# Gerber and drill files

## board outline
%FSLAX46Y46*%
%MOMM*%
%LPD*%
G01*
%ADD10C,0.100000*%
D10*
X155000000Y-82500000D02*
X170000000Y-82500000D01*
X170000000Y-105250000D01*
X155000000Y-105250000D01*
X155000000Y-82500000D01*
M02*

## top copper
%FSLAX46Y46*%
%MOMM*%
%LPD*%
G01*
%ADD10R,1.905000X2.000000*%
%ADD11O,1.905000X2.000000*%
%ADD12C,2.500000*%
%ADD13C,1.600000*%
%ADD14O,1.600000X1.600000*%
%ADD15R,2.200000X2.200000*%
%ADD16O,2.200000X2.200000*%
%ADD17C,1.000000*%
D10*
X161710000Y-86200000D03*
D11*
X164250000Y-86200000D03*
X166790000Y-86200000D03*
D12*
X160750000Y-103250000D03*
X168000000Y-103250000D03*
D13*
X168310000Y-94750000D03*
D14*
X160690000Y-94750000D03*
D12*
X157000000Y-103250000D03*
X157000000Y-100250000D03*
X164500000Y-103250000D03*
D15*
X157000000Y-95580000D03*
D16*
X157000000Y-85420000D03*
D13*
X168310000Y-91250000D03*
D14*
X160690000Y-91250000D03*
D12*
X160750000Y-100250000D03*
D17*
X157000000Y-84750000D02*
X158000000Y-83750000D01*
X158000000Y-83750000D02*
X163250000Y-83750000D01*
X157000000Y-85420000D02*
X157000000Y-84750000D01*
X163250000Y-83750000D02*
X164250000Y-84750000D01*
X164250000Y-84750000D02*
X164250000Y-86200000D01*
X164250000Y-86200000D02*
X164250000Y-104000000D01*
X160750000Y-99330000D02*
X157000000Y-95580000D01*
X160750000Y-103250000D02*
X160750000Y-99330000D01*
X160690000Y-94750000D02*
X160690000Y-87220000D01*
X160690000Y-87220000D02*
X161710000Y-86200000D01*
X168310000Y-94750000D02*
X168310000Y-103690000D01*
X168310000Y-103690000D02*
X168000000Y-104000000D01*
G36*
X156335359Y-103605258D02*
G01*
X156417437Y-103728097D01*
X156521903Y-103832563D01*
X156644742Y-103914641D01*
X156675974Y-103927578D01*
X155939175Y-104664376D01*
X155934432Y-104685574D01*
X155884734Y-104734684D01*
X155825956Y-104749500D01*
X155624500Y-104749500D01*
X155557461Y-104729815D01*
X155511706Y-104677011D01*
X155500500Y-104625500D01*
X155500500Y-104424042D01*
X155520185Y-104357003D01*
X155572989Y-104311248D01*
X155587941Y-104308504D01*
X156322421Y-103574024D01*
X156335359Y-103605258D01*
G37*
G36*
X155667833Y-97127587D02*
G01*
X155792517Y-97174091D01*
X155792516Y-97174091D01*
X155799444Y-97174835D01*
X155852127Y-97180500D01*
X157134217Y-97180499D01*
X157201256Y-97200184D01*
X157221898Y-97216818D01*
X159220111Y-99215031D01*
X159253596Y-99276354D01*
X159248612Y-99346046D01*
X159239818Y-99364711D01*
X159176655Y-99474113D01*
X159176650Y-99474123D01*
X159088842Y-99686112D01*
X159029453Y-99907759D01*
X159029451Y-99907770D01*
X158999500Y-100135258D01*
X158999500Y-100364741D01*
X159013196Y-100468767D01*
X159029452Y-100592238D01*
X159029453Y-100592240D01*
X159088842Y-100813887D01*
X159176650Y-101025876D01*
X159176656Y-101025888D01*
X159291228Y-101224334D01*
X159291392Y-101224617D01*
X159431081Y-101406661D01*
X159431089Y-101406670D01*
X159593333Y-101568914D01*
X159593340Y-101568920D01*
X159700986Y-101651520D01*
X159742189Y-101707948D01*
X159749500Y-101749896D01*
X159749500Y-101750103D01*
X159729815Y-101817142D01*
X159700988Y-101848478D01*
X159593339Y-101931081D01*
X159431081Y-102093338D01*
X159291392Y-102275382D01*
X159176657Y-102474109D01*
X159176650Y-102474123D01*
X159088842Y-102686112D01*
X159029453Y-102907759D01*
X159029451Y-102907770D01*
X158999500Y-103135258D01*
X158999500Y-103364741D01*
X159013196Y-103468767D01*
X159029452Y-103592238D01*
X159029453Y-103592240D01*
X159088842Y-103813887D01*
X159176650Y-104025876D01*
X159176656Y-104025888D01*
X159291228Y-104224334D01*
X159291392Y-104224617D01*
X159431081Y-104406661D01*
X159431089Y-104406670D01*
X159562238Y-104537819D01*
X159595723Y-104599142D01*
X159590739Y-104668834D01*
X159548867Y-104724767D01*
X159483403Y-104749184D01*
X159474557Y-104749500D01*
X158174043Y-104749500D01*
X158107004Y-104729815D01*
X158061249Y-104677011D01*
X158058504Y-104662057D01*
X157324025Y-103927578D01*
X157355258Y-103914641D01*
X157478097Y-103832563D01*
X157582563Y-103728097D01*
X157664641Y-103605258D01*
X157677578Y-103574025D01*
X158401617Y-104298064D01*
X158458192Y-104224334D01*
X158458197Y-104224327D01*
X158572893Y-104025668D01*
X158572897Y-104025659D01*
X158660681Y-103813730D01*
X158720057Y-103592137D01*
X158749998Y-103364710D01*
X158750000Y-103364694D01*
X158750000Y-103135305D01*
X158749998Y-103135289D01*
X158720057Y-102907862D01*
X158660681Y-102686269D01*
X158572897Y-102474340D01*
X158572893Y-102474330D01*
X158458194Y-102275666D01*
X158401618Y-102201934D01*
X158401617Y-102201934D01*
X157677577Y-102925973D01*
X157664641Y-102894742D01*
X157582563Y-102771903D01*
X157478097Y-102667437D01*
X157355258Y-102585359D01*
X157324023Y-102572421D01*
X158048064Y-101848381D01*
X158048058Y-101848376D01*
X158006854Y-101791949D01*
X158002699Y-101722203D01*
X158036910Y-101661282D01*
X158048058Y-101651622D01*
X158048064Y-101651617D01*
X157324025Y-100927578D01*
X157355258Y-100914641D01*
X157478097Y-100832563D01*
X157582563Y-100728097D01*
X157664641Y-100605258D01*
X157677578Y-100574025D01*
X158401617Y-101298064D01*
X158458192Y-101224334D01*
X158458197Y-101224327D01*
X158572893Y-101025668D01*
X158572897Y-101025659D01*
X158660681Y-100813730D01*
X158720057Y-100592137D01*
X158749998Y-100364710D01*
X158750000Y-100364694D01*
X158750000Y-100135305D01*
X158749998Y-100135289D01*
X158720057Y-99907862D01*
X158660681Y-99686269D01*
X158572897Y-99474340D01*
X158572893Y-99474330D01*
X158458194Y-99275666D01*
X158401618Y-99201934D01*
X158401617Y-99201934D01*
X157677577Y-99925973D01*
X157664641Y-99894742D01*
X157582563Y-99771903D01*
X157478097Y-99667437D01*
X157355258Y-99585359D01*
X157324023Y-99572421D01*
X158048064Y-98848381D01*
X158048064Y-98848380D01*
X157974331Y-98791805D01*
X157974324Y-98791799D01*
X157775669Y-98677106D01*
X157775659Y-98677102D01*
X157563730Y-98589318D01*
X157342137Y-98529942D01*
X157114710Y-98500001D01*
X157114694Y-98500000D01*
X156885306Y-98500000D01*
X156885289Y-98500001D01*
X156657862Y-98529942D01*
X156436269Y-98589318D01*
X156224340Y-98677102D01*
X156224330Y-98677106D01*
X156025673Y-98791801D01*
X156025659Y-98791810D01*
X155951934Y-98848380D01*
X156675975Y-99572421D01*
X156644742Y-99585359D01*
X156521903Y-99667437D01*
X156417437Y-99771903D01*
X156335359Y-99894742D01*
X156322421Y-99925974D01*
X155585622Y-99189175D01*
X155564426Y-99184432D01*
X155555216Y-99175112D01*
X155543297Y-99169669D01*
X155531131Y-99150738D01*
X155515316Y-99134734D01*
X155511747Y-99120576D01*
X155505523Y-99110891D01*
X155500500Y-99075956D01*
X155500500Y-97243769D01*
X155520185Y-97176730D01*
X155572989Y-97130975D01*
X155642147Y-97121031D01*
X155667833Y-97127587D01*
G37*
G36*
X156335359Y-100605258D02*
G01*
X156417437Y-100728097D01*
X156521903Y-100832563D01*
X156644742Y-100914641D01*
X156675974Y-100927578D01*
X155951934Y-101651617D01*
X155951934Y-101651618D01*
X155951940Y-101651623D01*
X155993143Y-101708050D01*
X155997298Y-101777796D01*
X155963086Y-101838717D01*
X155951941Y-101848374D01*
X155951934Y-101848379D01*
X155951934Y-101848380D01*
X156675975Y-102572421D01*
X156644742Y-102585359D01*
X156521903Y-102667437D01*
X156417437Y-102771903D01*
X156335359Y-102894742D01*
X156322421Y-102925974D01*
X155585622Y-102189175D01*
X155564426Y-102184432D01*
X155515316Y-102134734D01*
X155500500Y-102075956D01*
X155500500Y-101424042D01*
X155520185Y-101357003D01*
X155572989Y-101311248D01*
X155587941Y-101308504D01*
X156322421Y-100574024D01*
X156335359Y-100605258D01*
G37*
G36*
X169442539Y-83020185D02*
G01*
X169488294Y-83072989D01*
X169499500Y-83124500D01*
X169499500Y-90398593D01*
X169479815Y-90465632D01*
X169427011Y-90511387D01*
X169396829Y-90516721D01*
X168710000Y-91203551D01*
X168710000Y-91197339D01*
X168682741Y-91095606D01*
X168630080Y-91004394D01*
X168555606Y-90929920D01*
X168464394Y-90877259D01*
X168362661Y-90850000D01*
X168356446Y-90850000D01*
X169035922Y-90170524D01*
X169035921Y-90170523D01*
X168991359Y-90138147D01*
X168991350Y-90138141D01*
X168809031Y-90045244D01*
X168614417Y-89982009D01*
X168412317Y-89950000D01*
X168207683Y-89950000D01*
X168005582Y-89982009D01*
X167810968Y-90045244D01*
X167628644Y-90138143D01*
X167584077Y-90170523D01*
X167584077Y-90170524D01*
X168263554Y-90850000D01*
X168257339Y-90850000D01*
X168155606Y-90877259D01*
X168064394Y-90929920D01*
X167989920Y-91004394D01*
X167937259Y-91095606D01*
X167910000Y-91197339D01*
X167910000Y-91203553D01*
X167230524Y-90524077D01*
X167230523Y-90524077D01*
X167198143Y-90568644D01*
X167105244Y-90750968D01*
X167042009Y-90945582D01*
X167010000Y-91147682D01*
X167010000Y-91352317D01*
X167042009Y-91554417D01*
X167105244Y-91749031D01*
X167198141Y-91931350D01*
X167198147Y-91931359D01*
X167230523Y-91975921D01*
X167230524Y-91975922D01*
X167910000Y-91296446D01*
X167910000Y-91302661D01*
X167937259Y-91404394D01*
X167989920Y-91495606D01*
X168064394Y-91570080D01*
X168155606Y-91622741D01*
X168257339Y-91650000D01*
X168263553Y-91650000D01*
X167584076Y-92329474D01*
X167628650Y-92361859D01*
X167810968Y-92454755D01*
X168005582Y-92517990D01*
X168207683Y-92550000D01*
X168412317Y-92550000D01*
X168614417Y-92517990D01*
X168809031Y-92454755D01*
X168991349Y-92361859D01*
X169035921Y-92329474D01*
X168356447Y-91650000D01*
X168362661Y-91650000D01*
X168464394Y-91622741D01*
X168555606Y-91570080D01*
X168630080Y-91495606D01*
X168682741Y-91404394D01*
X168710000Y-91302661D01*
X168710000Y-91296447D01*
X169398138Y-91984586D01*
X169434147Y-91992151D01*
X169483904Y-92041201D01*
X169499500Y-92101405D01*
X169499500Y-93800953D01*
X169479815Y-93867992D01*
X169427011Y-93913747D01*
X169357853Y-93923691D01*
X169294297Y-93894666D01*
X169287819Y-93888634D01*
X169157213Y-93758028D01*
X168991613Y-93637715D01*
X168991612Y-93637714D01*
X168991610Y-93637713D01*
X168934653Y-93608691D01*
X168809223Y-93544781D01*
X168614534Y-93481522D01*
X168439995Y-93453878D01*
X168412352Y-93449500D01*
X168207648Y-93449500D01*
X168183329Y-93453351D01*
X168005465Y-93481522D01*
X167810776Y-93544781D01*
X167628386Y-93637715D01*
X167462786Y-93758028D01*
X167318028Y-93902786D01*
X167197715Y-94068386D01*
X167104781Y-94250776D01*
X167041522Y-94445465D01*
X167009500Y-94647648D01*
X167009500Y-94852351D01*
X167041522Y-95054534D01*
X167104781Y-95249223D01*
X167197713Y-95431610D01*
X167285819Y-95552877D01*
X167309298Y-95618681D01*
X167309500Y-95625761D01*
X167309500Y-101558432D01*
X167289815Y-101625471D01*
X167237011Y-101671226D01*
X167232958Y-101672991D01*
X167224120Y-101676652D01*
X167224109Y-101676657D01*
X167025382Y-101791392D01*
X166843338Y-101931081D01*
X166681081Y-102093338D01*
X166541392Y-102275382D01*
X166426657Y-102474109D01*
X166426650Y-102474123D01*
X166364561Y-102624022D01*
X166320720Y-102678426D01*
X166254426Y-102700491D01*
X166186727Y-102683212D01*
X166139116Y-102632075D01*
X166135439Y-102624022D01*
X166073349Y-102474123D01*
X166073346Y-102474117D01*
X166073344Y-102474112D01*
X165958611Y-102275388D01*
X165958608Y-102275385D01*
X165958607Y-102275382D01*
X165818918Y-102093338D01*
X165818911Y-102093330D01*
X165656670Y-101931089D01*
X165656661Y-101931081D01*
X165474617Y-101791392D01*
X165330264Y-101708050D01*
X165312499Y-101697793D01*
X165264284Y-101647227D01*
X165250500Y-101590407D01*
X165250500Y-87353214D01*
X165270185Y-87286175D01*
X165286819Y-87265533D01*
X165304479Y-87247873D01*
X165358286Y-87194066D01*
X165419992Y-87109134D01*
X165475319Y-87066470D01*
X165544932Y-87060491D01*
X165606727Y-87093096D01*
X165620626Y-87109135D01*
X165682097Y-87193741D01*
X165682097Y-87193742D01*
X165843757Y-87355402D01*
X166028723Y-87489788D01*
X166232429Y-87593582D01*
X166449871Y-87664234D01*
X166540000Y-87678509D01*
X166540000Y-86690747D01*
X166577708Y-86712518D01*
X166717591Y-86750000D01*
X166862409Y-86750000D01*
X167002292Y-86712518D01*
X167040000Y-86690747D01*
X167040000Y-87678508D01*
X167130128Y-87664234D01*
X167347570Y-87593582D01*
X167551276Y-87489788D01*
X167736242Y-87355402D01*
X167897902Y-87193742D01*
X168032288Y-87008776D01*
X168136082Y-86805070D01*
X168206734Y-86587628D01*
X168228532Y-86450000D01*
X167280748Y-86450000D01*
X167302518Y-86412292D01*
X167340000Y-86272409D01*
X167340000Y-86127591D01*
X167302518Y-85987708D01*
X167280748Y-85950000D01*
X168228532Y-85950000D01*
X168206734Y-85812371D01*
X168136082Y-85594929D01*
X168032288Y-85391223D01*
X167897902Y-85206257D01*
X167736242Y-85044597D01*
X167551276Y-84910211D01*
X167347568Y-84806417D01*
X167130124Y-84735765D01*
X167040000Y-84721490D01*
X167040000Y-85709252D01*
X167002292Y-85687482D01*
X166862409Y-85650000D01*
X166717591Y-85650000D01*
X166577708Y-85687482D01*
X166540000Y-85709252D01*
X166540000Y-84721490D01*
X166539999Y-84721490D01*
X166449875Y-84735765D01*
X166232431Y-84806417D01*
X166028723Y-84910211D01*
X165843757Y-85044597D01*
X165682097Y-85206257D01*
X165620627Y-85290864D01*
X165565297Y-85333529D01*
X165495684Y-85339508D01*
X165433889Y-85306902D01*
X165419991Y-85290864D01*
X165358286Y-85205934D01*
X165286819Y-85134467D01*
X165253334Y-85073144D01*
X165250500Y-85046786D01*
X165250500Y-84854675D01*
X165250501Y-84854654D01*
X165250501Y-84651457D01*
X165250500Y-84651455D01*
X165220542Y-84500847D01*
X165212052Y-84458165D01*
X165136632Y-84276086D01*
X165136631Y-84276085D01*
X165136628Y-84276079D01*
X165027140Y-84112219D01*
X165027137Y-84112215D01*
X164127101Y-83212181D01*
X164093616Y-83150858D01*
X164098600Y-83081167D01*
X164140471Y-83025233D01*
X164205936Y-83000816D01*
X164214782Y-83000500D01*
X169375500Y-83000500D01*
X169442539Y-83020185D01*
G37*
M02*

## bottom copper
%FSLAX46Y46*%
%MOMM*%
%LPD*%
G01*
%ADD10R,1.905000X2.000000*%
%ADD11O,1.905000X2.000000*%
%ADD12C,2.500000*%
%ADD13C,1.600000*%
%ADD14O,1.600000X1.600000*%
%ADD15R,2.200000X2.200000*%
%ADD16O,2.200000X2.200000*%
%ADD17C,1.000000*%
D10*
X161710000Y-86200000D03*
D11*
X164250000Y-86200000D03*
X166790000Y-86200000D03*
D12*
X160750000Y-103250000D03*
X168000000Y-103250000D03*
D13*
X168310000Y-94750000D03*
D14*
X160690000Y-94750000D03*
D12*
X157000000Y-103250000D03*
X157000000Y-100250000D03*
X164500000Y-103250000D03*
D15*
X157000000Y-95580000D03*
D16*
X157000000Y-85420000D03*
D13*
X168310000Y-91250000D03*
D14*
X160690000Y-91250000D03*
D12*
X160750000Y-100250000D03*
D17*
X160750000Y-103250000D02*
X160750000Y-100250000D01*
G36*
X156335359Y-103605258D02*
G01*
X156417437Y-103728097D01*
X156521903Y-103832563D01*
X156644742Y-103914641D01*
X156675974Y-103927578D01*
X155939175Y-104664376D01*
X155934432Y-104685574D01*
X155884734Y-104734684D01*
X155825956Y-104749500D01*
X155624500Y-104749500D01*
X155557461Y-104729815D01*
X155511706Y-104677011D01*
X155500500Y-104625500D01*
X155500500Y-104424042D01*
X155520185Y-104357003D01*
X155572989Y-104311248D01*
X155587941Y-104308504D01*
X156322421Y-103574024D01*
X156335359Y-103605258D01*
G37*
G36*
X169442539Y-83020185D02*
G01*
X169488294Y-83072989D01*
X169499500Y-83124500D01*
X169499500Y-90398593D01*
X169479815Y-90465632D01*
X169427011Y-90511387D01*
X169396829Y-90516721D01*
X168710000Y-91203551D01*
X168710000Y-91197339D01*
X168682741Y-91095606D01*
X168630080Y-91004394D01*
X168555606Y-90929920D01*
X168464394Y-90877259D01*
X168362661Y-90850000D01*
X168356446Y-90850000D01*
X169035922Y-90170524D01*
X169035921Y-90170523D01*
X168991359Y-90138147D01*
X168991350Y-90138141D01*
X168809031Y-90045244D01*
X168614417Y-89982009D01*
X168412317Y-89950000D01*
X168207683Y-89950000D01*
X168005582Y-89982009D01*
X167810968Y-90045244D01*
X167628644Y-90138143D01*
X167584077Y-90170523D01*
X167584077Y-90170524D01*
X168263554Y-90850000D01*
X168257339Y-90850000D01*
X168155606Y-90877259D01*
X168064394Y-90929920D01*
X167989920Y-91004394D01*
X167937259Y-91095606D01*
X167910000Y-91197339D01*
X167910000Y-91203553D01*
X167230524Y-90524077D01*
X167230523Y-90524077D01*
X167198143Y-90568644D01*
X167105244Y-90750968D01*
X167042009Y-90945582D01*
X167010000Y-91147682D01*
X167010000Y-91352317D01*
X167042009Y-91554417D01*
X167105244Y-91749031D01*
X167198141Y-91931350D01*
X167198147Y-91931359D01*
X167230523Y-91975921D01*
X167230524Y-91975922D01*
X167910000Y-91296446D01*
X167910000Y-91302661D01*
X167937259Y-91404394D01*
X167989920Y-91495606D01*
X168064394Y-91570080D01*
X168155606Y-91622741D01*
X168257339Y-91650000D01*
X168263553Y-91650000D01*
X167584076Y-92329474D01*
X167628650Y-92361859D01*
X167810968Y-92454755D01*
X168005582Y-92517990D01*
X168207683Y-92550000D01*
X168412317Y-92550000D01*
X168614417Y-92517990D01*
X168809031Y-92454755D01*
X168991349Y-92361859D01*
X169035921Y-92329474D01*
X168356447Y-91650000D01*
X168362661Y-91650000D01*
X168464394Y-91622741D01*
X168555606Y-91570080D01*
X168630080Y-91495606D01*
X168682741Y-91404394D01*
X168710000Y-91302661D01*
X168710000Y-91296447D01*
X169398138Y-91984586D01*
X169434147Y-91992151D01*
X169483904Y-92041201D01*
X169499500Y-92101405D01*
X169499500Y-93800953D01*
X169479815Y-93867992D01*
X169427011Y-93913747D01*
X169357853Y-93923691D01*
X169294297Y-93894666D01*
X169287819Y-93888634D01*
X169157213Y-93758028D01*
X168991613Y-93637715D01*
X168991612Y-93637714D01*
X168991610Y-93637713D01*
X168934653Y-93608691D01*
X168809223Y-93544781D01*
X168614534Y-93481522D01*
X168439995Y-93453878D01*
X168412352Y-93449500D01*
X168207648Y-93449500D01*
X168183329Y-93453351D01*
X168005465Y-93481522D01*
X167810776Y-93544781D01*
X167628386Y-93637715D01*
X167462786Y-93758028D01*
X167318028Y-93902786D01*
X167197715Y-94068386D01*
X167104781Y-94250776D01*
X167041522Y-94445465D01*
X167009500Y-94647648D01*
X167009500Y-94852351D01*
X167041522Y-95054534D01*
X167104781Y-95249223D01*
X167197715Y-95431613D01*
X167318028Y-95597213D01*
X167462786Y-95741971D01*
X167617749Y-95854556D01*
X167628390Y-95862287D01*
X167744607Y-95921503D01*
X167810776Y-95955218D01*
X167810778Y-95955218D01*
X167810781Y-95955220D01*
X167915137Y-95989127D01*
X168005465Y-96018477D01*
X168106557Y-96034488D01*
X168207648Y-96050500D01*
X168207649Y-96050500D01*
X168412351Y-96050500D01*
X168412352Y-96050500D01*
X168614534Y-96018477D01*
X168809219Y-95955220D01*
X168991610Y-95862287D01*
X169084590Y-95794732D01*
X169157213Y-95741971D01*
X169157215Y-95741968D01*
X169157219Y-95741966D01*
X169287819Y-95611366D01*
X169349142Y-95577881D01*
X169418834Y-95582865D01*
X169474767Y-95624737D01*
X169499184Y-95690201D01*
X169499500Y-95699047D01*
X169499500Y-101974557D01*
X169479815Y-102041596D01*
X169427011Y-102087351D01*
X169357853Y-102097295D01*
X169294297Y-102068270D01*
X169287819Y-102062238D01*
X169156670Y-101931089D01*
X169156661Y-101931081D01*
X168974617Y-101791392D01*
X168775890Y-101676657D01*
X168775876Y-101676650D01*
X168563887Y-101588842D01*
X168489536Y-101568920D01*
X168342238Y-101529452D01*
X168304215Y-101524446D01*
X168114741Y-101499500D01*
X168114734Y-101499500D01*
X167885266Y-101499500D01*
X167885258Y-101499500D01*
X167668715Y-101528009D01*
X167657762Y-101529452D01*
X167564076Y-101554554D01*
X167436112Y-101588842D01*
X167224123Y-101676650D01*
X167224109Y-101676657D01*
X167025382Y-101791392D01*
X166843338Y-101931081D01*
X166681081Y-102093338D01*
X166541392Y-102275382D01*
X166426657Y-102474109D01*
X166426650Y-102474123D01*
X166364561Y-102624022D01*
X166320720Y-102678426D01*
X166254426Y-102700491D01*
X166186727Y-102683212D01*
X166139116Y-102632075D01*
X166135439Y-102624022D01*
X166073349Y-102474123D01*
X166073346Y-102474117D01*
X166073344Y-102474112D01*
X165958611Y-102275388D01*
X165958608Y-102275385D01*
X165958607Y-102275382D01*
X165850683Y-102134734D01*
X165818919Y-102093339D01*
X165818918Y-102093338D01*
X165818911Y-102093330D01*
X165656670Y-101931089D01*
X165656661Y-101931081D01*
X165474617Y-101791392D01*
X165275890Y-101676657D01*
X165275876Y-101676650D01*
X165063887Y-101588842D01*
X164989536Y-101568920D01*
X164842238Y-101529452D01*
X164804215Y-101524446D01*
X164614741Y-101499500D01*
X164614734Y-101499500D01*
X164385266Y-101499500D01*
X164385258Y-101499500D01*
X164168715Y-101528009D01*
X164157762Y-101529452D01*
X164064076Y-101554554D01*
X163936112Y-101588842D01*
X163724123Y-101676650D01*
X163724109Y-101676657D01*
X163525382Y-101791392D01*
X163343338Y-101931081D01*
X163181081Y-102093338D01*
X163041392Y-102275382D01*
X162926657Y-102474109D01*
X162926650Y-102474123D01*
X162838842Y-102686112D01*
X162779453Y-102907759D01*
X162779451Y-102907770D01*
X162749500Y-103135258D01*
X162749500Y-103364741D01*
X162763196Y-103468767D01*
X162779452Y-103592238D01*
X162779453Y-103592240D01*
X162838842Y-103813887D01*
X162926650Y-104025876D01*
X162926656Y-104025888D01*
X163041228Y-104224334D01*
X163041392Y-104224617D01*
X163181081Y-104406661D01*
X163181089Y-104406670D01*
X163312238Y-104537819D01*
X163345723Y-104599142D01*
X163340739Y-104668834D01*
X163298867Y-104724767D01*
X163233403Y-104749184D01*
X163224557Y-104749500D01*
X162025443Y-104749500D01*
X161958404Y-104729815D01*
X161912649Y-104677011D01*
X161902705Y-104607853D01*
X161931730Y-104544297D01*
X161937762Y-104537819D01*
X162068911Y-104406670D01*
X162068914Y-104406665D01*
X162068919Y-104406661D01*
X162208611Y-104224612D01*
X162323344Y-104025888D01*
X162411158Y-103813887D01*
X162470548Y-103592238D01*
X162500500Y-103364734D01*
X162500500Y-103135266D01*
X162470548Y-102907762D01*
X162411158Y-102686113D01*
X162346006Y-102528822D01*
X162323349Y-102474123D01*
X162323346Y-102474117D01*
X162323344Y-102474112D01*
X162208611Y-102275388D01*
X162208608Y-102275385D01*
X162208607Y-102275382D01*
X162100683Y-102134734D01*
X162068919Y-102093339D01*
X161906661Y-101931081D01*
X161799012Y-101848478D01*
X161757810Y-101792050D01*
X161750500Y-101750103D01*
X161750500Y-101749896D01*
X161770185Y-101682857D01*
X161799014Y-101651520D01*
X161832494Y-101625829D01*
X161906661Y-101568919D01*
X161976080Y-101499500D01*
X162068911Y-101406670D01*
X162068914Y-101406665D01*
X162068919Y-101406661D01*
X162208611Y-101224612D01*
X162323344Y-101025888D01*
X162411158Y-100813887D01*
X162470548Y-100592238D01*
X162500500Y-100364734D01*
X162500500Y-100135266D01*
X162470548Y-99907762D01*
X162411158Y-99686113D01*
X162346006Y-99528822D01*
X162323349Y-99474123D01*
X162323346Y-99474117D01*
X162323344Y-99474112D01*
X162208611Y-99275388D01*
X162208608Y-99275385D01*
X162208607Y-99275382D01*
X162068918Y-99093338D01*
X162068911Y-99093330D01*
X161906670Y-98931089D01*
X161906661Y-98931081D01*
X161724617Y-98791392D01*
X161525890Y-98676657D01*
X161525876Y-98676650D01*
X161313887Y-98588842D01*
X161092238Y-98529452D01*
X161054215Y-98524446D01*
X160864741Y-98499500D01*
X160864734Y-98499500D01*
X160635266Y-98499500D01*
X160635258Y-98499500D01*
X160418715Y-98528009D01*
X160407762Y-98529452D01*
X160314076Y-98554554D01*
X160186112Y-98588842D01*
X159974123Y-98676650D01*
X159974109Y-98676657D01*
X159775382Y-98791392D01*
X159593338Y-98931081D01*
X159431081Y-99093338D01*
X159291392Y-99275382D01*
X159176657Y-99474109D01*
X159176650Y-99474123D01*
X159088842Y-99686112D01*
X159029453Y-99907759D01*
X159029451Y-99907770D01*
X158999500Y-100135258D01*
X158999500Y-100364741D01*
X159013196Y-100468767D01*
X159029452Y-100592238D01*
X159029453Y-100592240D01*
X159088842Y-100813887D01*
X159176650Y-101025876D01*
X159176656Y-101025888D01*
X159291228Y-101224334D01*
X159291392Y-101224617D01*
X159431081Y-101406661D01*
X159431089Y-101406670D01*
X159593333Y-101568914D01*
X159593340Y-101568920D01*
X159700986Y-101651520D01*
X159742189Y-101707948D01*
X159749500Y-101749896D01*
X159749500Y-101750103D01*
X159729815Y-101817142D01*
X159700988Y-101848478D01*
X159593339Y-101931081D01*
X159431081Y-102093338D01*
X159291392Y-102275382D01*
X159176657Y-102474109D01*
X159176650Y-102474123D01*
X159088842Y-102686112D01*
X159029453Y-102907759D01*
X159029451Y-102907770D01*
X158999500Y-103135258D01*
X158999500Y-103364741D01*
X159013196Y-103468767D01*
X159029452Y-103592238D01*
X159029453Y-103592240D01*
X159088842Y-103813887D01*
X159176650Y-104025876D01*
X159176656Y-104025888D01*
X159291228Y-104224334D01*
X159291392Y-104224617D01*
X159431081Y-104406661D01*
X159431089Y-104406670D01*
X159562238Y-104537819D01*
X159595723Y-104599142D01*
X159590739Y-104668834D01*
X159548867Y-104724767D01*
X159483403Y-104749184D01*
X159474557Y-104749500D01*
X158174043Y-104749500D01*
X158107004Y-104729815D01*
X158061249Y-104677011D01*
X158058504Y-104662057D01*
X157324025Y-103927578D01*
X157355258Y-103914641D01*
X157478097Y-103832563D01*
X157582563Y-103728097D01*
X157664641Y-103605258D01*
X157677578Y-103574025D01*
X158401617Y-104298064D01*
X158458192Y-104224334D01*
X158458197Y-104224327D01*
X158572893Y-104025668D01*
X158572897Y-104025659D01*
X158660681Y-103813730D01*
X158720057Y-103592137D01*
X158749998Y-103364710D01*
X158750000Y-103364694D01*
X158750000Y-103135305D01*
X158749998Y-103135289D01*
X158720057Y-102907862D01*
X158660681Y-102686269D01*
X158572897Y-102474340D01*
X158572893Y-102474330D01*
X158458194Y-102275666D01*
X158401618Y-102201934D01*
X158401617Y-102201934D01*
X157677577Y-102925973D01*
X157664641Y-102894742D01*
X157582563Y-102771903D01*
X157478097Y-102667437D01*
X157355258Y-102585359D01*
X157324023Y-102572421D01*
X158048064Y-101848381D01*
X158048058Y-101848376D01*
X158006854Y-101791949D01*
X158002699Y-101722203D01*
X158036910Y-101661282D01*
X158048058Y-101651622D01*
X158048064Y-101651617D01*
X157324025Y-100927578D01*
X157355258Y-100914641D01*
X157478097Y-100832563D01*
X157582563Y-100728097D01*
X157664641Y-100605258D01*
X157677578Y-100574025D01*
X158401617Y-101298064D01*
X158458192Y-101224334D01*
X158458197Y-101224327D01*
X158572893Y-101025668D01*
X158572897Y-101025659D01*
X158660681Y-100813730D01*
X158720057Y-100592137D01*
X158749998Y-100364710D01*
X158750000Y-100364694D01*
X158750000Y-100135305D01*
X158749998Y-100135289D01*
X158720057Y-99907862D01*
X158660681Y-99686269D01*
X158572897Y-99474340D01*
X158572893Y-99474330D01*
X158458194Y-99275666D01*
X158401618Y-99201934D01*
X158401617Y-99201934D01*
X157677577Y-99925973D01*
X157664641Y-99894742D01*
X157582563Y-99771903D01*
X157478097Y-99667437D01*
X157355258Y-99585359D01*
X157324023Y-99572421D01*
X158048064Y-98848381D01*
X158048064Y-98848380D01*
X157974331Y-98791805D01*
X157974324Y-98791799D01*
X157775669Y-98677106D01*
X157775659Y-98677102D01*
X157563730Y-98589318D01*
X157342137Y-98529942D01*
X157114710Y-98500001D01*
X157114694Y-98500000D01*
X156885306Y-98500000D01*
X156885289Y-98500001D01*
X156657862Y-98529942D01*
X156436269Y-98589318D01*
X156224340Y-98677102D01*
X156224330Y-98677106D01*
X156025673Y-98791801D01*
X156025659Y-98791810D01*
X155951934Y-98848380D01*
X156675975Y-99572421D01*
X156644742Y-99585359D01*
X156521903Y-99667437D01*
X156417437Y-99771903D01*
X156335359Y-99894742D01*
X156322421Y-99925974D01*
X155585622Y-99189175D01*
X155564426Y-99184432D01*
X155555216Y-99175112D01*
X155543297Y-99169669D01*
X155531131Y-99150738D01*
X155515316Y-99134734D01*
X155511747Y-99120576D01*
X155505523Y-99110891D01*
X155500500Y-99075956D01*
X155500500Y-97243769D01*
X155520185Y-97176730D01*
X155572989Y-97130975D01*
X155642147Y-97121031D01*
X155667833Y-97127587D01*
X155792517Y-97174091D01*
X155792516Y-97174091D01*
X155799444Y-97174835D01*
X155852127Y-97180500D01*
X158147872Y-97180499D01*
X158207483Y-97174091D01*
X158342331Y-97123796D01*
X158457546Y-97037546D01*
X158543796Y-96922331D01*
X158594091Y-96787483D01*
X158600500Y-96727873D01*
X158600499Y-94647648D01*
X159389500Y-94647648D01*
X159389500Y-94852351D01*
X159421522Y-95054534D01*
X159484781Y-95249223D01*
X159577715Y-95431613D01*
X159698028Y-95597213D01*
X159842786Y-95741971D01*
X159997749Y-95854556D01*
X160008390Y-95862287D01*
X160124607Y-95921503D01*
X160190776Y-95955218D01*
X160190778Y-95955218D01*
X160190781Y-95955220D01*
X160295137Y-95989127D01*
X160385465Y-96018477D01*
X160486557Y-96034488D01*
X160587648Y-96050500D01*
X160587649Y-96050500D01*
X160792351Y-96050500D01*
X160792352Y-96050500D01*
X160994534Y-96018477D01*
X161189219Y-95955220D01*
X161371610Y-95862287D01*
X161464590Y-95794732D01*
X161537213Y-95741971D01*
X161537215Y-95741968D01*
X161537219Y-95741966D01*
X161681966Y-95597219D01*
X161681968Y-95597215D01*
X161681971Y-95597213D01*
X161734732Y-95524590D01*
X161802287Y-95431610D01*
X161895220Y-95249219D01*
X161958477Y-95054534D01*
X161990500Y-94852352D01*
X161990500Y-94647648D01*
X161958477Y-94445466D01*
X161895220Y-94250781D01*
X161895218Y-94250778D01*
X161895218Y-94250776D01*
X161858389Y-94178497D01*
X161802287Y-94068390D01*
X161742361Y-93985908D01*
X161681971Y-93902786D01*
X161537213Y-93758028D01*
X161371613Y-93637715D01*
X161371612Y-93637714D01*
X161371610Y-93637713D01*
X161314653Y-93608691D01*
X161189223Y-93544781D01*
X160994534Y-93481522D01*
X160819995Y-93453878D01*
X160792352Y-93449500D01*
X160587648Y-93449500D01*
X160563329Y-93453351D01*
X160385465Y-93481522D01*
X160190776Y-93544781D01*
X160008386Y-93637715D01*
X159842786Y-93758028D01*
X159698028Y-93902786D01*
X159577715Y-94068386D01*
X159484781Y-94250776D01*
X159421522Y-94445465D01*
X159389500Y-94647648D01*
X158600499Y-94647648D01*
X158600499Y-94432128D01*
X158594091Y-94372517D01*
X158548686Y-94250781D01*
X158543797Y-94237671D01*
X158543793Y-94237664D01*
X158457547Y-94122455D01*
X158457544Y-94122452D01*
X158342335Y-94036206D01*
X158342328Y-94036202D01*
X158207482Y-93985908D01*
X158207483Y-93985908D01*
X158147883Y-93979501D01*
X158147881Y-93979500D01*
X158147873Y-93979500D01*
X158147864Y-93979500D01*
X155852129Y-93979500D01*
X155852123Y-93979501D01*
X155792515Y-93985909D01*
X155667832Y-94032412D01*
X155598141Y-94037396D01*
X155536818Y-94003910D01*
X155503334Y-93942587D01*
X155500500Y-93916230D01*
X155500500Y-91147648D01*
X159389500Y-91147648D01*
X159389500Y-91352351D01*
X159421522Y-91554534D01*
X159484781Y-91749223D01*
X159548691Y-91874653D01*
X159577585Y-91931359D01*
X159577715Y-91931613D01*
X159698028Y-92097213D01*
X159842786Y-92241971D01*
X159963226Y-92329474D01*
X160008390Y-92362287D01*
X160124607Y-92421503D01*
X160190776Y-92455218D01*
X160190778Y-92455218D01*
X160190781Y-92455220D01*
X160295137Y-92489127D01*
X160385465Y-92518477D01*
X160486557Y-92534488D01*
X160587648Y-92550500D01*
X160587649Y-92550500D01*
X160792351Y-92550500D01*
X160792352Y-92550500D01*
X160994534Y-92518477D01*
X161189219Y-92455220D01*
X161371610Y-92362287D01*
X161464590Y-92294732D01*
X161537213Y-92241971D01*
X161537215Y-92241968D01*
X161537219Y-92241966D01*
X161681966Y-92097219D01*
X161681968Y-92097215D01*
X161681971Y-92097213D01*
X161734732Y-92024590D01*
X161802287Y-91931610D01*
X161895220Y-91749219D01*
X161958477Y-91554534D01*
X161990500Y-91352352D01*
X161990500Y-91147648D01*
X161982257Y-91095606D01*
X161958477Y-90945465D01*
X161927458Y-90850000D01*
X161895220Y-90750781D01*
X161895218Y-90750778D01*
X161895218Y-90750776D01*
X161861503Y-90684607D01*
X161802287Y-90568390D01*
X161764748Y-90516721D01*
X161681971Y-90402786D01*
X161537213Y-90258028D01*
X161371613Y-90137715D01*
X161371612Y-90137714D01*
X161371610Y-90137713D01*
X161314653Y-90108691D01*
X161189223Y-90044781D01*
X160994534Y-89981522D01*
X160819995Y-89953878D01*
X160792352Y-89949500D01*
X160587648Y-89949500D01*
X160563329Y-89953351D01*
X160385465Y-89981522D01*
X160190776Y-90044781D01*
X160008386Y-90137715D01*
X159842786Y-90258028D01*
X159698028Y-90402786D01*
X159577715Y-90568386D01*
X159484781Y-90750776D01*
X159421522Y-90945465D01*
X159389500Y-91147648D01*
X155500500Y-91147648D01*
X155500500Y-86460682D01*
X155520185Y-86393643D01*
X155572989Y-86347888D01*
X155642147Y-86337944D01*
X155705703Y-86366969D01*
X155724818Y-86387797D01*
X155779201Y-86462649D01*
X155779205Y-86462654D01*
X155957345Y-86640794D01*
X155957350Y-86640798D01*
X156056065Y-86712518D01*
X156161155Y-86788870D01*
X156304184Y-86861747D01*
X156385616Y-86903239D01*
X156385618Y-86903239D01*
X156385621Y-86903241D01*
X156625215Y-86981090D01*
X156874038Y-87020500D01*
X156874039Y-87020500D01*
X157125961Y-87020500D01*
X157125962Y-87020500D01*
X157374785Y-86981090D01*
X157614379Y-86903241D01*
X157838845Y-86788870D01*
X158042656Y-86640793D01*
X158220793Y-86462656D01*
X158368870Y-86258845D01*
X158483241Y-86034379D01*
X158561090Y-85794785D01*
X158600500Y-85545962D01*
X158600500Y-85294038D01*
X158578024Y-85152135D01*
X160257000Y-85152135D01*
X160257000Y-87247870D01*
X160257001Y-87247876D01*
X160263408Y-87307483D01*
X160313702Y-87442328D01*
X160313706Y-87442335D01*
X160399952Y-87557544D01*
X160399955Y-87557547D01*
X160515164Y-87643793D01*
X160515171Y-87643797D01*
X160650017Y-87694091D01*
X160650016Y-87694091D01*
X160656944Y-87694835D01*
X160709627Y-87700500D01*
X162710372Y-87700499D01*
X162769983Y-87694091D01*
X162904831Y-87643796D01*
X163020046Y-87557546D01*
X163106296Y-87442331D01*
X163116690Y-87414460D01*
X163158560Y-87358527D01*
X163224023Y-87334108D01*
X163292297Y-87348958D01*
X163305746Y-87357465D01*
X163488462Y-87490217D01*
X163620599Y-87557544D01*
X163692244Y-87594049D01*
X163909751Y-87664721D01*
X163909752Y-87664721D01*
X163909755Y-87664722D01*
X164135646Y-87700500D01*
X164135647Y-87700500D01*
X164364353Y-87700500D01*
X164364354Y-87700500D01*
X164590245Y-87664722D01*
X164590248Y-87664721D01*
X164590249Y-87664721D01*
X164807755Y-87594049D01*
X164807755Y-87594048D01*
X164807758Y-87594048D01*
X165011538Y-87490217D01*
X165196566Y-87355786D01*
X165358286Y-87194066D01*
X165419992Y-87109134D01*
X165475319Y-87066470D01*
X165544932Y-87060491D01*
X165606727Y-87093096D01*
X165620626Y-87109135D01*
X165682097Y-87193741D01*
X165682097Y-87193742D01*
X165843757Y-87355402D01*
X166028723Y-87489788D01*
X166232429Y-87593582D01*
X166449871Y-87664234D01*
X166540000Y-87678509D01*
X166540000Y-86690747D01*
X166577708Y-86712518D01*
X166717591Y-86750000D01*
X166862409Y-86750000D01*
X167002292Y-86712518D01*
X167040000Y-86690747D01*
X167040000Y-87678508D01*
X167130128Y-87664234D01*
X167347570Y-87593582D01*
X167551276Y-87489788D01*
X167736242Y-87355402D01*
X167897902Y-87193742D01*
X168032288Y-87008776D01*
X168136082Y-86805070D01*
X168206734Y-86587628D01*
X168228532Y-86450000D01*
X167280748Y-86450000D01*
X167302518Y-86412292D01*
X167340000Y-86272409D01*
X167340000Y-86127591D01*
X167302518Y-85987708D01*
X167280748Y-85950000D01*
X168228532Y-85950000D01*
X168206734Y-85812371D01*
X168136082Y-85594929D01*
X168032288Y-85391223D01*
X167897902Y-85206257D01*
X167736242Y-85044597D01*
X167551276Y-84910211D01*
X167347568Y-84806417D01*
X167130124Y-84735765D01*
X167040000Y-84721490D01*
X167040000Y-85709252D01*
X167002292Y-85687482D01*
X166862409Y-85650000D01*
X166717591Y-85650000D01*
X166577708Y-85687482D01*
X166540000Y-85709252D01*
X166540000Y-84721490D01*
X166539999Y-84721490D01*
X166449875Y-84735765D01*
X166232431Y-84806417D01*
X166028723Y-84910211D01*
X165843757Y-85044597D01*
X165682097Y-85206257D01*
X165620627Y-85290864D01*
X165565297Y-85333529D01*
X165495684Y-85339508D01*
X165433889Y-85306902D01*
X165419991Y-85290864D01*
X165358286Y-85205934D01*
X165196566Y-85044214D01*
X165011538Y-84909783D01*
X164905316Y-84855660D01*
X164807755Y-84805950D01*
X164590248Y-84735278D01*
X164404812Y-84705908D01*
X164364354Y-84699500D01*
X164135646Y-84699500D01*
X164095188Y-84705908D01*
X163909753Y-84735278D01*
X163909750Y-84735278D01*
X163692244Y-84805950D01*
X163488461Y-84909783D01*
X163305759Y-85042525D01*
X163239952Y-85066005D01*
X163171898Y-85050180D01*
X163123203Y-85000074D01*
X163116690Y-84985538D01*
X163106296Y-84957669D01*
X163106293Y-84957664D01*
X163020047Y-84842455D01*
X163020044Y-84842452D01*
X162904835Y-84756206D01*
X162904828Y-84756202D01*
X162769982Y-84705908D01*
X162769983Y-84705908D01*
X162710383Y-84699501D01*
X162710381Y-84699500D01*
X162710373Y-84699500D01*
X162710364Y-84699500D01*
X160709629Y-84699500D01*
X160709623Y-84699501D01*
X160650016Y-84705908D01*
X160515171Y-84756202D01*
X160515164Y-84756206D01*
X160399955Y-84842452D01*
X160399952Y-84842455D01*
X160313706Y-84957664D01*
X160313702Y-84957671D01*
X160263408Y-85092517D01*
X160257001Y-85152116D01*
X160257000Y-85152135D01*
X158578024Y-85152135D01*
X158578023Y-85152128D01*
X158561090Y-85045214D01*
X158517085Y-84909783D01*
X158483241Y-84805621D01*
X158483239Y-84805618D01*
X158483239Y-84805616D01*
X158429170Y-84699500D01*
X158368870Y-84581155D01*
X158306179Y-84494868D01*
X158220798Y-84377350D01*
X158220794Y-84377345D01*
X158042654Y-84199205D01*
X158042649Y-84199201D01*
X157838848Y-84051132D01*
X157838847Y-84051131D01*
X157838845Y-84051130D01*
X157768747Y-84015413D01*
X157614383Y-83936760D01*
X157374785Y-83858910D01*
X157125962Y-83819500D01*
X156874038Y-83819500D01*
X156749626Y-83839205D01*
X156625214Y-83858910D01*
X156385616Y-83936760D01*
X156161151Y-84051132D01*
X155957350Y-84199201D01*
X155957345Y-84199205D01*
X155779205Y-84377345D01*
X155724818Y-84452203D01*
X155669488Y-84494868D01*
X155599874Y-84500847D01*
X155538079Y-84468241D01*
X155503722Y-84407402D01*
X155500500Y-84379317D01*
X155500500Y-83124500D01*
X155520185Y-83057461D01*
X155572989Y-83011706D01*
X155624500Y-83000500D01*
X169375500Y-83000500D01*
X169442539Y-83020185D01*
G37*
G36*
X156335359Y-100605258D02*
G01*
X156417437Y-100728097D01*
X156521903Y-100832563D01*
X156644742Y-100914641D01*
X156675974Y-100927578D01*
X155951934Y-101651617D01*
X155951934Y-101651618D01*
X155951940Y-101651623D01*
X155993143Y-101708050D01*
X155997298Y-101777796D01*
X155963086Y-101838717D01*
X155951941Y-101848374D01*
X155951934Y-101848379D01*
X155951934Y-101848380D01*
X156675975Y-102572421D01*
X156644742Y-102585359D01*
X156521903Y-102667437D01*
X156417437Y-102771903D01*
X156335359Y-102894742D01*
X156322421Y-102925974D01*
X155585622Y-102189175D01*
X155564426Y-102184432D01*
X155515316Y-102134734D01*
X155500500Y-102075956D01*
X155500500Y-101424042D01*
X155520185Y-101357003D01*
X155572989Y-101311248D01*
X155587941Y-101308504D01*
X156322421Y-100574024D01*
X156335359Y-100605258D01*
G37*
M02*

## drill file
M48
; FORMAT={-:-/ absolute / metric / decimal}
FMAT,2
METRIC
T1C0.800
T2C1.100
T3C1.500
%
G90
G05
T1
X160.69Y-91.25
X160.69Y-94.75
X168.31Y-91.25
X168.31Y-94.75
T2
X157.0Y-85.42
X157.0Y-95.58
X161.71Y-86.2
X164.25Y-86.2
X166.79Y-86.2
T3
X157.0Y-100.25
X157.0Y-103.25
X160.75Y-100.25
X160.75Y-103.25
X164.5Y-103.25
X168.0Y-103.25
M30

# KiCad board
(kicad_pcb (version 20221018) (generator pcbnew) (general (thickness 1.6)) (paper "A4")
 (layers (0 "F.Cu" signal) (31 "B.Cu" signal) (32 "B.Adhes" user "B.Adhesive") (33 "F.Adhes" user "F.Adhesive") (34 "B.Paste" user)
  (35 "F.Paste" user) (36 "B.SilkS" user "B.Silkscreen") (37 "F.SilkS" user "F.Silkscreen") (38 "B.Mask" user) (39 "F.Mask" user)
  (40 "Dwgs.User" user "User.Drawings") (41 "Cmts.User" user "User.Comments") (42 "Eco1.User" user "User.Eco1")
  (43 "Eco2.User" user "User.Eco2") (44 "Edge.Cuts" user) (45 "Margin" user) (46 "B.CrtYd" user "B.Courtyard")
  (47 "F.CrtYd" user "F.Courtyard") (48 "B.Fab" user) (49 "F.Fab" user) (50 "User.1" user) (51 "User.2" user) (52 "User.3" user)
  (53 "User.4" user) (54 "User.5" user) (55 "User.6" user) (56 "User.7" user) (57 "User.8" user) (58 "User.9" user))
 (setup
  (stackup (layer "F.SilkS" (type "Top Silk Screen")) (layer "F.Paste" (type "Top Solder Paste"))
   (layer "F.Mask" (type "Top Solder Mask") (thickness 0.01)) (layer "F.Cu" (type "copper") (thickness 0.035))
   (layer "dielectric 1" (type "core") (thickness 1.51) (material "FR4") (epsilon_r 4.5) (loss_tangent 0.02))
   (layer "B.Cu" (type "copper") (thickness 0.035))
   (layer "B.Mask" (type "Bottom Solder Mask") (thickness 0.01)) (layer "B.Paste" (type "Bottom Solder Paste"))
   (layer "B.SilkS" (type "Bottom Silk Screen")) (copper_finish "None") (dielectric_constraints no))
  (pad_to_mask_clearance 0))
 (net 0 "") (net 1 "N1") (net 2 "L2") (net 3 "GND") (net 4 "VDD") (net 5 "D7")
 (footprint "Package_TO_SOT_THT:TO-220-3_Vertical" (layer "F.Cu") (at 161.71 86.2)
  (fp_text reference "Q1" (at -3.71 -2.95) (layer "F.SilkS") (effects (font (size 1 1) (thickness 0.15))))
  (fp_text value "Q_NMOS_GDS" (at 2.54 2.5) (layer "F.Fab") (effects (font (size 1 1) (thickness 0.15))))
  (pad "1" thru_hole rect (at 0 0) (size 1.905 2) (drill 1.1) (layers "*.Cu" "*.Mask") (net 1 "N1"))
  (pad "2" thru_hole oval (at 2.54 0) (size 1.905 2) (drill 1.1) (layers "*.Cu" "*.Mask") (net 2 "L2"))
  (pad "3" thru_hole oval (at 5.08 0) (size 1.905 2) (drill 1.1) (layers "*.Cu" "*.Mask") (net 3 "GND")))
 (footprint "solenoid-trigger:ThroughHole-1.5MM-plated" (layer "F.Cu") (at 160.75 103.25)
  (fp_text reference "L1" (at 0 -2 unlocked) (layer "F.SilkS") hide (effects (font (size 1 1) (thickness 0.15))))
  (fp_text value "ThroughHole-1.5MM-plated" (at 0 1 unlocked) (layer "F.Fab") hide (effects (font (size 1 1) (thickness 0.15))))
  (pad "1" thru_hole circle (at 0 0) (size 2.5 2.5) (drill 1.5) (layers "*.Cu" "*.Mask") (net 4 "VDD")))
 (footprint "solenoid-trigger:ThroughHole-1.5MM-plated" (layer "F.Cu") (at 168 103.25)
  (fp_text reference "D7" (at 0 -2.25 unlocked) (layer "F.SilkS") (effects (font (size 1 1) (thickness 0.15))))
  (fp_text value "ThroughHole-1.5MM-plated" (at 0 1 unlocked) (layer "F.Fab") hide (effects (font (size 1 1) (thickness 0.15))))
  (pad "1" thru_hole circle (at 0 0) (size 2.5 2.5) (drill 1.5) (layers "*.Cu" "*.Mask") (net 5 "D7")))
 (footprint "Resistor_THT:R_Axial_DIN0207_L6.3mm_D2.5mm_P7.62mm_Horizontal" (layer "F.Cu") (at 168.31 94.75 180)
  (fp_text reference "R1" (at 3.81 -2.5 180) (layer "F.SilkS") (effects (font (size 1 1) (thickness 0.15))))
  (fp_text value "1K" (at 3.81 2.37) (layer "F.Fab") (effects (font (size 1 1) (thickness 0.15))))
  (pad "1" thru_hole circle (at 0 0 180) (size 1.6 1.6) (drill 0.8) (layers "*.Cu" "*.Mask") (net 5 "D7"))
  (pad "2" thru_hole oval (at 7.62 0 180) (size 1.6 1.6) (drill 0.8) (layers "*.Cu" "*.Mask") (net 1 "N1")))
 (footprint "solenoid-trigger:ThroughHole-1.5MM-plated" (layer "F.Cu") (at 157 103.25)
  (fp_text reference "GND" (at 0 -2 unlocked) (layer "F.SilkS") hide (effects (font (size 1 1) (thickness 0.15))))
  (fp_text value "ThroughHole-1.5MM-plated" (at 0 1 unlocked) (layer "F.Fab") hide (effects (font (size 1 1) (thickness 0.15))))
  (pad "1" thru_hole circle (at 0 0) (size 2.5 2.5) (drill 1.5) (layers "*.Cu" "*.Mask") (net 3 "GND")))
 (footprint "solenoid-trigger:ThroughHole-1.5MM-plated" (layer "F.Cu") (at 157 100.25)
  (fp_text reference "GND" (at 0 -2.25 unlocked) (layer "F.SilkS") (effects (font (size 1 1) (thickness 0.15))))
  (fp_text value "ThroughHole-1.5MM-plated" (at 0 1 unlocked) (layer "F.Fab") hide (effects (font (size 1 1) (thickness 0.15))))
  (pad "1" thru_hole circle (at 0 0) (size 2.5 2.5) (drill 1.5) (layers "*.Cu" "*.Mask") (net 3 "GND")))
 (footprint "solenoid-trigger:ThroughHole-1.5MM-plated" (layer "F.Cu") (at 164.5 103.25)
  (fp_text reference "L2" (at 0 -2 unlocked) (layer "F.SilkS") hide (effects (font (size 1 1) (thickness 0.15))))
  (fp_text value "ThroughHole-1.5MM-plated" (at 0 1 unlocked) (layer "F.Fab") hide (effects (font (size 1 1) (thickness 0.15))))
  (pad "1" thru_hole circle (at 0 0) (size 2.5 2.5) (drill 1.5) (layers "*.Cu" "*.Mask") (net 2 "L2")))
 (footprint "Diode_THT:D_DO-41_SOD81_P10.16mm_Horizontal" (layer "F.Cu") (at 157 95.58 90)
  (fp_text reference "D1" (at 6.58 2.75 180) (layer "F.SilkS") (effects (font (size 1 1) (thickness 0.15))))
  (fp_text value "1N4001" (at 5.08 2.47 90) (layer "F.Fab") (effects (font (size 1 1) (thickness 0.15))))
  (pad "1" thru_hole rect (at 0 0 90) (size 2.2 2.2) (drill 1.1) (layers "*.Cu" "*.Mask") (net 4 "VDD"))
  (pad "2" thru_hole oval (at 10.16 0 90) (size 2.2 2.2) (drill 1.1) (layers "*.Cu" "*.Mask") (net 2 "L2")))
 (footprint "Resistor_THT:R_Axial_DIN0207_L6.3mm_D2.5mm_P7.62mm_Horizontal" (layer "F.Cu") (at 168.31 91.25 180)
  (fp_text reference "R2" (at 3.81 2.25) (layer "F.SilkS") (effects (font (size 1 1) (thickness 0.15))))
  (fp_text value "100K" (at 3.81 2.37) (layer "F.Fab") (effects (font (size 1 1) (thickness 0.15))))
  (pad "1" thru_hole circle (at 0 0 180) (size 1.6 1.6) (drill 0.8) (layers "*.Cu" "*.Mask") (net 3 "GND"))
  (pad "2" thru_hole oval (at 7.62 0 180) (size 1.6 1.6) (drill 0.8) (layers "*.Cu" "*.Mask") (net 1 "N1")))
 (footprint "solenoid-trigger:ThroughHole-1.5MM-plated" (layer "F.Cu") (at 160.75 100.25)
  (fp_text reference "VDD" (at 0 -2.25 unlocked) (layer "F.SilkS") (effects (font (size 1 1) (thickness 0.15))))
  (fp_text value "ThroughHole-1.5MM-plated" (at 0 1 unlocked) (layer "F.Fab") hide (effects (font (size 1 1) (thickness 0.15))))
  (pad "1" thru_hole circle (at 0 0) (size 2.5 2.5) (drill 1.5) (layers "*.Cu" "*.Mask") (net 4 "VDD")))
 (gr_rect (start 155 82.5) (end 170 105.25) (stroke (width 0.1) (type default)) (fill none) (layer "Edge.Cuts"))
 (segment (start 157 84.75) (end 158 83.75) (width 1) (layer "F.Cu") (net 2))
 (segment (start 158 83.75) (end 163.25 83.75) (width 1) (layer "F.Cu") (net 2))
 (segment (start 157 85.42) (end 157 84.75) (width 1) (layer "F.Cu") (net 2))
 (segment (start 163.25 83.75) (end 164.25 84.75) (width 1) (layer "F.Cu") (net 2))
 (segment (start 164.25 84.75) (end 164.25 86.2) (width 1) (layer "F.Cu") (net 2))
 (segment (start 164.25 86.2) (end 164.25 104) (width 1) (layer "F.Cu") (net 2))
 (segment (start 160.75 99.33) (end 157 95.58) (width 1) (layer "F.Cu") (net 4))
 (segment (start 160.75 103.25) (end 160.75 99.33) (width 1) (layer "F.Cu") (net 4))
 (segment (start 160.75 103.25) (end 160.75 100.25) (width 1) (layer "B.Cu") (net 4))
 (segment (start 160.69 94.75) (end 160.69 87.22) (width 1) (layer "F.Cu") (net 1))
 (segment (start 160.69 87.22) (end 161.71 86.2) (width 1) (layer "F.Cu") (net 1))
 (segment (start 168.31 94.75) (end 168.31 103.69) (width 1) (layer "F.Cu") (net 5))
 (segment (start 168.31 103.69) (end 168 104) (width 1) (layer "F.Cu") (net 5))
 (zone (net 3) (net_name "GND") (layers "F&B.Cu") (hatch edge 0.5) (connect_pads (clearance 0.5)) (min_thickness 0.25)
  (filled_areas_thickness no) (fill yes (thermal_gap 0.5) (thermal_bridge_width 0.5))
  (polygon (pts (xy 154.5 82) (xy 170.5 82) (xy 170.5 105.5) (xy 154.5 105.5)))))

